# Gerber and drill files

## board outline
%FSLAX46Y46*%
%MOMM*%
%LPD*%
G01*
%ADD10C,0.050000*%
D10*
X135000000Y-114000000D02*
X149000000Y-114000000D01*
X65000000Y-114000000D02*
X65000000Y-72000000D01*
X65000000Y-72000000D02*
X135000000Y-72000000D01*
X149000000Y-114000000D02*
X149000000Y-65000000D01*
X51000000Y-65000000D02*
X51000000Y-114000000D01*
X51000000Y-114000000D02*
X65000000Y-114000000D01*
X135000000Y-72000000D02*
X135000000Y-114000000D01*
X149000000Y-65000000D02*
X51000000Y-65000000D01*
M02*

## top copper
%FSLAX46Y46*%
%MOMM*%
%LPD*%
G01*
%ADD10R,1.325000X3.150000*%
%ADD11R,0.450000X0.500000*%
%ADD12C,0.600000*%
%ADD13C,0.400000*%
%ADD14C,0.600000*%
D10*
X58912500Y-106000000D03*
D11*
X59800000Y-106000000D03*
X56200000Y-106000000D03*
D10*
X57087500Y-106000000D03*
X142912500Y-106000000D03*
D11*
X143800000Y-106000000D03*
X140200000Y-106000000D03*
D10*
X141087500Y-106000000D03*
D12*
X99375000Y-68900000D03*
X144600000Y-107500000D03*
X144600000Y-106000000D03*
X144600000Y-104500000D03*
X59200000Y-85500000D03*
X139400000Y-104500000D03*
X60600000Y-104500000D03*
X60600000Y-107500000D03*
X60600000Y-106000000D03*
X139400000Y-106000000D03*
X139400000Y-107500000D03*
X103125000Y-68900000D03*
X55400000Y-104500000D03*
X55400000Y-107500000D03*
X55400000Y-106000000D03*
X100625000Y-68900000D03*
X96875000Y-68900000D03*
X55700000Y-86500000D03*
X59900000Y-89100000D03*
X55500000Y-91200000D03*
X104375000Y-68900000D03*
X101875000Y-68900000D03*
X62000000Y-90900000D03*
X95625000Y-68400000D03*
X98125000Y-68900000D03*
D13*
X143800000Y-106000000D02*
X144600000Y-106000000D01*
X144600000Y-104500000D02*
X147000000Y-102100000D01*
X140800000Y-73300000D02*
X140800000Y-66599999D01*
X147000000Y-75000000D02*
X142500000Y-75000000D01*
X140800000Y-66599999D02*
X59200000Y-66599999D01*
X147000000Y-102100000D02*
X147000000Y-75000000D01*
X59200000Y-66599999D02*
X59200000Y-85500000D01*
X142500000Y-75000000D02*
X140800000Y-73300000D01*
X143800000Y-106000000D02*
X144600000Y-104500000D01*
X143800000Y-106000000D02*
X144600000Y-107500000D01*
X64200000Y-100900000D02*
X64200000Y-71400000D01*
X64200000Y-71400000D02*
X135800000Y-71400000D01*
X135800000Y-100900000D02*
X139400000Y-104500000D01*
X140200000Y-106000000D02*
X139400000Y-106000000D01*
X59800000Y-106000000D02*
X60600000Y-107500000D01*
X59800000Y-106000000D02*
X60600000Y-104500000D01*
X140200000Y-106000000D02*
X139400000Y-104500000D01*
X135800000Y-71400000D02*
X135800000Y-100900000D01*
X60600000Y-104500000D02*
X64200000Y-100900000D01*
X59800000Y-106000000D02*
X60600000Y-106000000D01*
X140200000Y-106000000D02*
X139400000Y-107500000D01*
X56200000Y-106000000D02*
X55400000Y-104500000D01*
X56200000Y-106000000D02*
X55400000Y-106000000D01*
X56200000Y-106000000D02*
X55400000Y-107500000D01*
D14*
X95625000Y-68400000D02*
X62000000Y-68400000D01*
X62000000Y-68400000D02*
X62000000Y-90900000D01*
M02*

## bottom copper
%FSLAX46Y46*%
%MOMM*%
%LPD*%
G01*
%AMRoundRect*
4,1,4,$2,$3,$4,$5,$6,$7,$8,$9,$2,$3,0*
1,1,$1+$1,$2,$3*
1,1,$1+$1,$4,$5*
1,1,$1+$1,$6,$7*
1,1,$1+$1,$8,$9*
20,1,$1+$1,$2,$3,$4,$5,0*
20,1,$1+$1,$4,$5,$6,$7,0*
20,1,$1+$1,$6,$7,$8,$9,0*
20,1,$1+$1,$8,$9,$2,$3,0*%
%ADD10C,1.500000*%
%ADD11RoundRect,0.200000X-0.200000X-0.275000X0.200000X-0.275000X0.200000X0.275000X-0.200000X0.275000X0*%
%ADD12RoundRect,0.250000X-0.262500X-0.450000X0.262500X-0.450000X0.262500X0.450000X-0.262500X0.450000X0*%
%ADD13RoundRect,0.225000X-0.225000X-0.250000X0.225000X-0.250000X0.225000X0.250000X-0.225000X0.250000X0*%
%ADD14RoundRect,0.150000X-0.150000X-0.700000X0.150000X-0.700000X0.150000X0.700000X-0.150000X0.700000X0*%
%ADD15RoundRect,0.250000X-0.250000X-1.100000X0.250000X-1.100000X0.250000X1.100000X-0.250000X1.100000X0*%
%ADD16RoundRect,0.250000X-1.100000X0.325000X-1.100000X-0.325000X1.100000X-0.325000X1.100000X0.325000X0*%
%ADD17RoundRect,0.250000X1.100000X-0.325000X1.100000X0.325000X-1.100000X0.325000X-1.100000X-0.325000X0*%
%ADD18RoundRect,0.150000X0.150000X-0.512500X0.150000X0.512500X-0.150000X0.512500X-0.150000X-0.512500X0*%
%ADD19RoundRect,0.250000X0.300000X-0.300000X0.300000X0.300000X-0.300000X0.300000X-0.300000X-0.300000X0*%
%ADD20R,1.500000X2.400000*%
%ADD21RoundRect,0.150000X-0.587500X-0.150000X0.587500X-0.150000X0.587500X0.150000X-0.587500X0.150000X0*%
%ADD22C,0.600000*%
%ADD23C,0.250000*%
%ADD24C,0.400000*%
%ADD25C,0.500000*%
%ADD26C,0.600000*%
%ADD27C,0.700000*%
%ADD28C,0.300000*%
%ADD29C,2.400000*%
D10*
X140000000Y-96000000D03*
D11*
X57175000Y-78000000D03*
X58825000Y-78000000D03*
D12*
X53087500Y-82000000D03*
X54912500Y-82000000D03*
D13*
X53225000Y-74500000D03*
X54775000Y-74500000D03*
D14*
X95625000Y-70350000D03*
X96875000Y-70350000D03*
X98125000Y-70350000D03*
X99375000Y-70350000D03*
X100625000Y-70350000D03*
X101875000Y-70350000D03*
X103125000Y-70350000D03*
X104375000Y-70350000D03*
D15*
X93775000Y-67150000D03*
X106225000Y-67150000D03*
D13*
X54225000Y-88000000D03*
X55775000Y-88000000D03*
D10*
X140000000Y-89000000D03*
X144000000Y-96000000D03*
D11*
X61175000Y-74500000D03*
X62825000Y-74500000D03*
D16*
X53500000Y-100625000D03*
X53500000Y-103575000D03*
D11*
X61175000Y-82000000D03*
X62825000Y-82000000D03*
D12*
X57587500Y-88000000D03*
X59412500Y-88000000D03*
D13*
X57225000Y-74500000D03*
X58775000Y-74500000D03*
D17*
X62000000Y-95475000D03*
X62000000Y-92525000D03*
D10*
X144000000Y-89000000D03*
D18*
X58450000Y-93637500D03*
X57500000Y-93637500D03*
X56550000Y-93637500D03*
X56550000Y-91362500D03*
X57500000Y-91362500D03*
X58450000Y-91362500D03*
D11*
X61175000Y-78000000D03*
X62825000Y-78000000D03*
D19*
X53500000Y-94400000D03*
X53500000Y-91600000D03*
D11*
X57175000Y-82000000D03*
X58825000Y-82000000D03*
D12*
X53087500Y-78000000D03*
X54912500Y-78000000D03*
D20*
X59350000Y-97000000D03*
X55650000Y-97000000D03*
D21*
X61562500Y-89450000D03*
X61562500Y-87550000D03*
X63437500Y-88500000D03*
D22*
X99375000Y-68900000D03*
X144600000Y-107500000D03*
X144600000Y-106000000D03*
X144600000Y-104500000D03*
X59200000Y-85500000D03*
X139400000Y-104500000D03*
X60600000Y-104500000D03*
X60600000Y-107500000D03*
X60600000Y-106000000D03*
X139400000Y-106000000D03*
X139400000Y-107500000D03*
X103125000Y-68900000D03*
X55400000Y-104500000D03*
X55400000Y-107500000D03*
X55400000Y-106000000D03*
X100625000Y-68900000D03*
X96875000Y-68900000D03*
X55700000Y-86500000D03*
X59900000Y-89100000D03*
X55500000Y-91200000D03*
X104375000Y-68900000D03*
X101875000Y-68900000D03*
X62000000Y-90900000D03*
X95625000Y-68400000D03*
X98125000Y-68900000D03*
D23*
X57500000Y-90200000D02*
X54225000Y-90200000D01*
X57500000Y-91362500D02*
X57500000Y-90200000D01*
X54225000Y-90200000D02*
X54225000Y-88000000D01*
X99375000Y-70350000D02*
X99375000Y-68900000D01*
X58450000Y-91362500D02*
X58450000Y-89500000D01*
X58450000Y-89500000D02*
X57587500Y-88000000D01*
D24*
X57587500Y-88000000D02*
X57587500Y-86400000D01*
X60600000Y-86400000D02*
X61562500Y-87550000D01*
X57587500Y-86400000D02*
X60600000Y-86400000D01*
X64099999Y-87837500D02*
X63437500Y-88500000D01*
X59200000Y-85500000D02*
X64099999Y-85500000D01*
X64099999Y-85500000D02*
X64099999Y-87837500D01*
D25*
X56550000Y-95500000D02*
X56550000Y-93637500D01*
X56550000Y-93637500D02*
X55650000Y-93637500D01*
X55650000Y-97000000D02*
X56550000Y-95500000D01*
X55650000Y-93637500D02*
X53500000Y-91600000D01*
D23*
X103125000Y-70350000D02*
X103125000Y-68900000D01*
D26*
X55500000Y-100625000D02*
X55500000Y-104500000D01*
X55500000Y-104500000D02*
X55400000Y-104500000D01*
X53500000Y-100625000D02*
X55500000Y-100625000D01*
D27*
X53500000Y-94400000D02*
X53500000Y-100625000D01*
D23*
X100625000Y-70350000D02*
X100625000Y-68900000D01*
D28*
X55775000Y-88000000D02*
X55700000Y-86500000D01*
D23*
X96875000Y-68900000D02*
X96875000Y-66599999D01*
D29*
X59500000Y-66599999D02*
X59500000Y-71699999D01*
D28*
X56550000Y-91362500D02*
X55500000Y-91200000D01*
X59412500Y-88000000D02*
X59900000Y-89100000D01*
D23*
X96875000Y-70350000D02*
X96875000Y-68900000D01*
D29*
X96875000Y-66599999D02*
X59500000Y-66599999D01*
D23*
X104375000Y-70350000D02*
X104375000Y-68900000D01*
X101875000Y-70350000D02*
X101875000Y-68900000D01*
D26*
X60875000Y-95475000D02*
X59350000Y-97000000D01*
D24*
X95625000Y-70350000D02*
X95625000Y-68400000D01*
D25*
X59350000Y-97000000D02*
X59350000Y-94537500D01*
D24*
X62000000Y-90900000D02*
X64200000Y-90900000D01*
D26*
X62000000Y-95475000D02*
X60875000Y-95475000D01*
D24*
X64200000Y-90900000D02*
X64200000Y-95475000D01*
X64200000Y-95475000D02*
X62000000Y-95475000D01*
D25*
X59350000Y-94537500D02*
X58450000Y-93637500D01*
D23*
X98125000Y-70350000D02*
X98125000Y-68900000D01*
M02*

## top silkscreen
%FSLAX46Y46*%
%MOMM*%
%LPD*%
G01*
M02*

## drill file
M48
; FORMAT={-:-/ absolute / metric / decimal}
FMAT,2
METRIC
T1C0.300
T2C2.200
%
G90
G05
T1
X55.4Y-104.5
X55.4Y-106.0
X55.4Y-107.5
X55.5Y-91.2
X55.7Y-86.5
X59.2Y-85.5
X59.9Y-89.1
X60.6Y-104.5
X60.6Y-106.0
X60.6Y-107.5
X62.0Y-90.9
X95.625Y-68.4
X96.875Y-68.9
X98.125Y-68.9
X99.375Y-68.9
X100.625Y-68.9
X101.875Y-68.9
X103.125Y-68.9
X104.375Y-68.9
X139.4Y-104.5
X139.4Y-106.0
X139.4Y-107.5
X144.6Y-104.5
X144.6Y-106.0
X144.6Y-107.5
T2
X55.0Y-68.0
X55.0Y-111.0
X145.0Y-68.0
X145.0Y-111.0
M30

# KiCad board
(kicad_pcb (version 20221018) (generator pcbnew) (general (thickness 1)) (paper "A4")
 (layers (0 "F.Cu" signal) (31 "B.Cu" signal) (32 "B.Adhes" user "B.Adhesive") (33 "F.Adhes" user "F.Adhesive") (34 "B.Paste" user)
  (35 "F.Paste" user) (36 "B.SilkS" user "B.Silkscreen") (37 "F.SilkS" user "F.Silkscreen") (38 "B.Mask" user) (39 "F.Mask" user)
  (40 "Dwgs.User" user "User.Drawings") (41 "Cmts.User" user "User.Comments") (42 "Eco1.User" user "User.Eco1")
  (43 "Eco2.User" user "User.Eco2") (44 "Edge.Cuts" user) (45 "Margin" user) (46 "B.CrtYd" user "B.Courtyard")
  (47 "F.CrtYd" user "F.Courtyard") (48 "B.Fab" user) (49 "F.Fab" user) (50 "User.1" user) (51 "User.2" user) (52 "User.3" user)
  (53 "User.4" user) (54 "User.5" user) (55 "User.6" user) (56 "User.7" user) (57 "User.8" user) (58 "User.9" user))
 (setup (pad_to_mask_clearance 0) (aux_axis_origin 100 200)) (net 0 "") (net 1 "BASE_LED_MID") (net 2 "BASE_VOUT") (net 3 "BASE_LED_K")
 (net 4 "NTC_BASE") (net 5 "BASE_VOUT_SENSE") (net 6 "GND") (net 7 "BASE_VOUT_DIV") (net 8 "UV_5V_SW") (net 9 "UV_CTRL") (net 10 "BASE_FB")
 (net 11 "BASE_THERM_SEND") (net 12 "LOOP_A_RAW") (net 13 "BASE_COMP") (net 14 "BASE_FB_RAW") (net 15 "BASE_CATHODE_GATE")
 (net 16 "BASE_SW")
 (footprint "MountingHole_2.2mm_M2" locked (layer "F.Cu") (at 55 68)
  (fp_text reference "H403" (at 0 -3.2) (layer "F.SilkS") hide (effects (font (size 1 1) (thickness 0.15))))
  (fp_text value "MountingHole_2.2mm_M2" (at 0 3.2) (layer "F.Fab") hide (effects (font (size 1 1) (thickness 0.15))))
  (pad "" np_thru_hole circle locked (at 0 0) (size 2.2 2.2) (drill 2.2) (layers "*.Cu" "*.Mask")))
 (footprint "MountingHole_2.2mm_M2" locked (layer "F.Cu") (at 145 111)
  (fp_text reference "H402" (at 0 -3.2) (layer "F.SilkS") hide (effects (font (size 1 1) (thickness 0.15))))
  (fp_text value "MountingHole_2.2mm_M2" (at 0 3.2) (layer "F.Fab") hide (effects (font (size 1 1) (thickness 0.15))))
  (pad "" np_thru_hole circle locked (at 0 0) (size 2.2 2.2) (drill 2.2) (layers "*.Cu" "*.Mask")))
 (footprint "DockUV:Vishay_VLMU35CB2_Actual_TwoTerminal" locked (layer "F.Cu") (at 58 106)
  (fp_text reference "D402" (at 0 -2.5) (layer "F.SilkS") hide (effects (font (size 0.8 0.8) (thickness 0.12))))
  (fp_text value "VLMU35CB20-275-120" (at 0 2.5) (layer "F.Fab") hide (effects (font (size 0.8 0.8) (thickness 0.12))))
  (pad "1" smd rect locked (at 0.9125 0) (size 1.325 3.15) (layers "F.Cu" "F.Paste" "F.Mask") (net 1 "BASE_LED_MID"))
  (pad "1" smd rect locked (at 1.8 0) (size 0.45 0.5) (layers "F.Cu" "F.Paste" "F.Mask") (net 1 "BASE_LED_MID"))
  (pad "2" smd rect locked (at -1.8 0) (size 0.45 0.5) (layers "F.Cu" "F.Paste" "F.Mask") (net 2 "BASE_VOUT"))
  (pad "2" smd rect locked (at -0.9125 0) (size 1.325 3.15) (layers "F.Cu" "F.Paste" "F.Mask") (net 2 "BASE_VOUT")))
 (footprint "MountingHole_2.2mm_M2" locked (layer "F.Cu") (at 55 111)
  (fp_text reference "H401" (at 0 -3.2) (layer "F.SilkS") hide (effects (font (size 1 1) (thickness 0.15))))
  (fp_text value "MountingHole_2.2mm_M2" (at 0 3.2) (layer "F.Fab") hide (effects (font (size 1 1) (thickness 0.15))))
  (pad "" np_thru_hole circle locked (at 0 0) (size 2.2 2.2) (drill 2.2) (layers "*.Cu" "*.Mask")))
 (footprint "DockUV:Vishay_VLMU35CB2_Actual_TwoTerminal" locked (layer "F.Cu") (at 142 106)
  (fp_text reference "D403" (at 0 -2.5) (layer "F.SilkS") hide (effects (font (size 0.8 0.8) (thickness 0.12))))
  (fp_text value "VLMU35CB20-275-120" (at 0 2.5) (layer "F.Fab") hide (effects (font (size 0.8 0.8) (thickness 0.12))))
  (pad "1" smd rect locked (at 0.9125 0) (size 1.325 3.15) (layers "F.Cu" "F.Paste" "F.Mask") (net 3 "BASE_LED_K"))
  (pad "1" smd rect locked (at 1.8 0) (size 0.45 0.5) (layers "F.Cu" "F.Paste" "F.Mask") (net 3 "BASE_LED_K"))
  (pad "2" smd rect locked (at -1.8 0) (size 0.45 0.5) (layers "F.Cu" "F.Paste" "F.Mask") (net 1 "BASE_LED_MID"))
  (pad "2" smd rect locked (at -0.9125 0) (size 1.325 3.15) (layers "F.Cu" "F.Paste" "F.Mask") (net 1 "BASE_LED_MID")))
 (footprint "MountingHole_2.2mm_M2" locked (layer "F.Cu") (at 145 68)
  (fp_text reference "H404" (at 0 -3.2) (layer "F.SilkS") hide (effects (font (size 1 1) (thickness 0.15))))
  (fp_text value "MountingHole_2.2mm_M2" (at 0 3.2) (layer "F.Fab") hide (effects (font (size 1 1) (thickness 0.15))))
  (pad "" np_thru_hole circle locked (at 0 0) (size 2.2 2.2) (drill 2.2) (layers "*.Cu" "*.Mask")))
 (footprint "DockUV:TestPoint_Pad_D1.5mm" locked (layer "B.Cu") (at 140 96)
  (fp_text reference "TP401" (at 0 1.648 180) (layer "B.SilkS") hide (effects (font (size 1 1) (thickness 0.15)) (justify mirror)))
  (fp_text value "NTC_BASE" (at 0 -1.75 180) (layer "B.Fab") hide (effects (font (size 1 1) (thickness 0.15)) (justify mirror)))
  (pad "1" smd circle locked (at 0 0) (size 1.5 1.5) (layers "B.Cu" "B.Mask") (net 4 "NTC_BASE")))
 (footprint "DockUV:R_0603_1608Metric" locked (layer "B.Cu") (at 58 78)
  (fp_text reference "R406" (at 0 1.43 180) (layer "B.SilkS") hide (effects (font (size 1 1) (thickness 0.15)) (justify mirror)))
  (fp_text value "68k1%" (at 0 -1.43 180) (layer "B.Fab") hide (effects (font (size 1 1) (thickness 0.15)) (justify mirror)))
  (pad "1" smd roundrect locked (at -0.825 0) (size 0.8 0.95) (layers "B.Cu" "B.Paste" "B.Mask") (roundrect_rratio 0.25)
   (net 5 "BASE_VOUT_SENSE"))
  (pad "2" smd roundrect locked (at 0.825 0) (size 0.8 0.95) (layers "B.Cu" "B.Paste" "B.Mask") (roundrect_rratio 0.25) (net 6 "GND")))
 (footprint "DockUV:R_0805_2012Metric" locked (layer "B.Cu") (at 54 82)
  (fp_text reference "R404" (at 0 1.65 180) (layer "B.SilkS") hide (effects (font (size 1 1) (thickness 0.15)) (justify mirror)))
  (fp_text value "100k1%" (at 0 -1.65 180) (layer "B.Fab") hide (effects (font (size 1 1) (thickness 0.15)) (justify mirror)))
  (pad "1" smd roundrect locked (at -0.9125 0) (size 1.025 1.4) (layers "B.Cu" "B.Paste" "B.Mask") (roundrect_rratio 0.243902)
   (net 2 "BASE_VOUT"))
  (pad "2" smd roundrect locked (at 0.9125 0) (size 1.025 1.4) (layers "B.Cu" "B.Paste" "B.Mask") (roundrect_rratio 0.243902) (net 6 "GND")))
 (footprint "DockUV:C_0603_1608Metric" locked (layer "B.Cu") (at 54 74.5)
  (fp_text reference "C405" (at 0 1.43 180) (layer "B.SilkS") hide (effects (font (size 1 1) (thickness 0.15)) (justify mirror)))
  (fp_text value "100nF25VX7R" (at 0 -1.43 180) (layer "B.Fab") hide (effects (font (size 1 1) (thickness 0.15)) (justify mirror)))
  (pad "1" smd roundrect locked (at -0.775 0) (size 0.9 0.95) (layers "B.Cu" "B.Paste" "B.Mask") (roundrect_rratio 0.25)
   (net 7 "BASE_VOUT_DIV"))
  (pad "2" smd roundrect locked (at 0.775 0) (size 0.9 0.95) (layers "B.Cu" "B.Paste" "B.Mask") (roundrect_rratio 0.25) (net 6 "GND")))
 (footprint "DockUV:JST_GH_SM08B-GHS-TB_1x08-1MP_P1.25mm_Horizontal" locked (layer "B.Cu") (at 100 68.5)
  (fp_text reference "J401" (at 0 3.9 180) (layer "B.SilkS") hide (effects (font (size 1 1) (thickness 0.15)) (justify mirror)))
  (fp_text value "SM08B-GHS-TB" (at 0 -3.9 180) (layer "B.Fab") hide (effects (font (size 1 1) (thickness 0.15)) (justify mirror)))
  (pad "1" smd roundrect locked (at -4.375 1.85) (size 0.6 1.7) (layers "B.Cu" "B.Paste" "B.Mask") (roundrect_rratio 0.25)
   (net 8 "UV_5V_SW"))
  (pad "2" smd roundrect locked (at -3.125 1.85) (size 0.6 1.7) (layers "B.Cu" "B.Paste" "B.Mask") (roundrect_rratio 0.25) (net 6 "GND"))
  (pad "3" smd roundrect locked (at -1.875 1.85) (size 0.6 1.7) (layers "B.Cu" "B.Paste" "B.Mask") (roundrect_rratio 0.25) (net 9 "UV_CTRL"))
  (pad "4" smd roundrect locked (at -0.625 1.85) (size 0.6 1.7) (layers "B.Cu" "B.Paste" "B.Mask") (roundrect_rratio 0.25)
   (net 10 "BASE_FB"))
  (pad "5" smd roundrect locked (at 0.625 1.85) (size 0.6 1.7) (layers "B.Cu" "B.Paste" "B.Mask") (roundrect_rratio 0.25)
   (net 7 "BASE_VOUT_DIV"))
  (pad "6" smd roundrect locked (at 1.875 1.85) (size 0.6 1.7) (layers "B.Cu" "B.Paste" "B.Mask") (roundrect_rratio 0.25) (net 4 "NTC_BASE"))
  (pad "7" smd roundrect locked (at 3.125 1.85) (size 0.6 1.7) (layers "B.Cu" "B.Paste" "B.Mask") (roundrect_rratio 0.25)
   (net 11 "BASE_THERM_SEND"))
  (pad "8" smd roundrect locked (at 4.375 1.85) (size 0.6 1.7) (layers "B.Cu" "B.Paste" "B.Mask") (roundrect_rratio 0.25)
   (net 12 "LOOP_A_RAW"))
  (pad "MP" smd roundrect locked (at -6.225 -1.35) (size 1 2.7) (layers "B.Cu" "B.Paste" "B.Mask") (roundrect_rratio 0.25) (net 6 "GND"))
  (pad "MP" smd roundrect locked (at 6.225 -1.35) (size 1 2.7) (layers "B.Cu" "B.Paste" "B.Mask") (roundrect_rratio 0.25) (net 6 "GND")))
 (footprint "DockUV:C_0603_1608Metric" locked (layer "B.Cu") (at 55 88)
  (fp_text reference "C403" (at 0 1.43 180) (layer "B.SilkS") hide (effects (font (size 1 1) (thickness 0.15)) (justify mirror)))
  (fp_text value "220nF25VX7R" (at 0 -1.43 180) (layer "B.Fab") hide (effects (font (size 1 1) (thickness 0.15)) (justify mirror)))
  (pad "1" smd roundrect locked (at -0.775 0) (size 0.9 0.95) (layers "B.Cu" "B.Paste" "B.Mask") (roundrect_rratio 0.25)
   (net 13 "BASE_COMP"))
  (pad "2" smd roundrect locked (at 0.775 0) (size 0.9 0.95) (layers "B.Cu" "B.Paste" "B.Mask") (roundrect_rratio 0.25) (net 6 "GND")))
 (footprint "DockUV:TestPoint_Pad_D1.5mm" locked (layer "B.Cu") (at 140 89)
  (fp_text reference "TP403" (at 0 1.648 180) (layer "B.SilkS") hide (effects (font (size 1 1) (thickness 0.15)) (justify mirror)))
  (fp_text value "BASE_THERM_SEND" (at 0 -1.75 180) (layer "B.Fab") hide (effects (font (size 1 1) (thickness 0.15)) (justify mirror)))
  (pad "1" smd circle locked (at 0 0) (size 1.5 1.5) (layers "B.Cu" "B.Mask") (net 11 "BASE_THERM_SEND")))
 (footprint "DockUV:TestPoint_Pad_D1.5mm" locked (layer "B.Cu") (at 144 96)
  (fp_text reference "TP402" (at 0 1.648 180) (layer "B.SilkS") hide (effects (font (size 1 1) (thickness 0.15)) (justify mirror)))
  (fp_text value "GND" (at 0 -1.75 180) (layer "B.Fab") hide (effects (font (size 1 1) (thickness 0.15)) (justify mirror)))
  (pad "1" smd circle locked (at 0 0) (size 1.5 1.5) (layers "B.Cu" "B.Mask") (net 6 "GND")))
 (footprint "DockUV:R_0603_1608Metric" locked (layer "B.Cu") (at 62 74.5)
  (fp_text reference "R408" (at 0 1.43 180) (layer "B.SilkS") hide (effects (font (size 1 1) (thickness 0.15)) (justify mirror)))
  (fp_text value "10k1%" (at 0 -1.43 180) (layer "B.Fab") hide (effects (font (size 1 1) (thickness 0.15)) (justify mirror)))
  (pad "1" smd roundrect locked (at -0.825 0) (size 0.8 0.95) (layers "B.Cu" "B.Paste" "B.Mask") (roundrect_rratio 0.25)
   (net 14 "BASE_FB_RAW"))
  (pad "2" smd roundrect locked (at 0.825 0) (size 0.8 0.95) (layers "B.Cu" "B.Paste" "B.Mask") (roundrect_rratio 0.25) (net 10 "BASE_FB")))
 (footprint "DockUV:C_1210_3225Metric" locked (layer "B.Cu") (at 53.5 102.1 -90)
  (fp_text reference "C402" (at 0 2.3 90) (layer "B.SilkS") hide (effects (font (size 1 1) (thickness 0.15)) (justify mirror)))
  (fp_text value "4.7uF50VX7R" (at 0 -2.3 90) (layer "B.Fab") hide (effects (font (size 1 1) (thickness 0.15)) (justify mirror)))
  (pad "1" smd roundrect locked (at -1.475 0 270) (size 1.15 2.7) (layers "B.Cu" "B.Paste" "B.Mask") (roundrect_rratio 0.217391)
   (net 2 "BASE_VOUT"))
  (pad "2" smd roundrect locked (at 1.475 0 270) (size 1.15 2.7) (layers "B.Cu" "B.Paste" "B.Mask") (roundrect_rratio 0.217391)
   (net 6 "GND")))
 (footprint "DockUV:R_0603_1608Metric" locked (layer "B.Cu") (at 62 82)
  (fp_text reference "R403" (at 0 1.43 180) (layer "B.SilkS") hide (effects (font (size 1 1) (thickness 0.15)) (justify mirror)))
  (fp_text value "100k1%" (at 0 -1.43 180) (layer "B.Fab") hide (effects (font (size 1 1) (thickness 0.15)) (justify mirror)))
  (pad "1" smd roundrect locked (at -0.825 0) (size 0.8 0.95) (layers "B.Cu" "B.Paste" "B.Mask") (roundrect_rratio 0.25)
   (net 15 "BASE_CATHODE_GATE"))
  (pad "2" smd roundrect locked (at 0.825 0) (size 0.8 0.95) (layers "B.Cu" "B.Paste" "B.Mask") (roundrect_rratio 0.25) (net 6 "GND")))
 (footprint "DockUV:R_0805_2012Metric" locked (layer "B.Cu") (at 58.5 88)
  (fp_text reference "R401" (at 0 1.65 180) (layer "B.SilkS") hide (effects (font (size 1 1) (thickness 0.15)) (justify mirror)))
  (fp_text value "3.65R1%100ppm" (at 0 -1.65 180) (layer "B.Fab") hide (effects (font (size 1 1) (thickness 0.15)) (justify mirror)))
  (pad "1" smd roundrect locked (at -0.9125 0) (size 1.025 1.4) (layers "B.Cu" "B.Paste" "B.Mask") (roundrect_rratio 0.243902)
   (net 14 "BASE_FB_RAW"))
  (pad "2" smd roundrect locked (at 0.9125 0) (size 1.025 1.4) (layers "B.Cu" "B.Paste" "B.Mask") (roundrect_rratio 0.243902) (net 6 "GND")))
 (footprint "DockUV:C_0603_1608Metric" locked (layer "B.Cu") (at 58 74.5)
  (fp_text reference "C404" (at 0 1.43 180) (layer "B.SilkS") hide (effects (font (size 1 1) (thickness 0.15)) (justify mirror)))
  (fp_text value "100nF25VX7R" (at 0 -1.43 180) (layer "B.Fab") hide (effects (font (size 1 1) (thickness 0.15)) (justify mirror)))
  (pad "1" smd roundrect locked (at -0.775 0) (size 0.9 0.95) (layers "B.Cu" "B.Paste" "B.Mask") (roundrect_rratio 0.25) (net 10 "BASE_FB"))
  (pad "2" smd roundrect locked (at 0.775 0) (size 0.9 0.95) (layers "B.Cu" "B.Paste" "B.Mask") (roundrect_rratio 0.25) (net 6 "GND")))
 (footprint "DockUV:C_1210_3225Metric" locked (layer "B.Cu") (at 62 94 90)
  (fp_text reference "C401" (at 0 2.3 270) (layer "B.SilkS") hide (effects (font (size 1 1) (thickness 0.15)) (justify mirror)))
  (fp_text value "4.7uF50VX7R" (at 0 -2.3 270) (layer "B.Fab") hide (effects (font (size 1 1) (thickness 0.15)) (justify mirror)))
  (pad "1" smd roundrect locked (at -1.475 0 90) (size 1.15 2.7) (layers "B.Cu" "B.Paste" "B.Mask") (roundrect_rratio 0.217391)
   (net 8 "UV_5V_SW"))
  (pad "2" smd roundrect locked (at 1.475 0 90) (size 1.15 2.7) (layers "B.Cu" "B.Paste" "B.Mask") (roundrect_rratio 0.217391) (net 6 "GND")))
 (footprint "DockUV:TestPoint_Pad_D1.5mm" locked (layer "B.Cu") (at 144 89)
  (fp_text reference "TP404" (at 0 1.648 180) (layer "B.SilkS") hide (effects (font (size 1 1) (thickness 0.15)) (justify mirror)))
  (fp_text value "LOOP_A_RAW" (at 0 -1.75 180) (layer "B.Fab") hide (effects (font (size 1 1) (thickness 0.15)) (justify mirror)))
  (pad "1" smd circle locked (at 0 0) (size 1.5 1.5) (layers "B.Cu" "B.Mask") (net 12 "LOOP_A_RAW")))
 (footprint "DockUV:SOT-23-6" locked (layer "B.Cu") (at 57.5 92.5 90)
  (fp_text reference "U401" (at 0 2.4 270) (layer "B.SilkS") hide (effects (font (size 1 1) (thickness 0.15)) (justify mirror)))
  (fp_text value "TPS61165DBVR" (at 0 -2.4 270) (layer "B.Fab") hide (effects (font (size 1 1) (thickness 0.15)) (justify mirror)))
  (pad "1" smd roundrect locked (at -1.1375 0.95 90) (size 1.325 0.6) (layers "B.Cu" "B.Paste" "B.Mask") (roundrect_rratio 0.25)
   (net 8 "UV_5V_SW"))
  (pad "2" smd roundrect locked (at -1.1375 0 90) (size 1.325 0.6) (layers "B.Cu" "B.Paste" "B.Mask") (roundrect_rratio 0.25)
   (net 9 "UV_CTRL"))
  (pad "3" smd roundrect locked (at -1.1375 -0.95 90) (size 1.325 0.6) (layers "B.Cu" "B.Paste" "B.Mask") (roundrect_rratio 0.25)
   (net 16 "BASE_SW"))
  (pad "4" smd roundrect locked (at 1.1375 -0.95 90) (size 1.325 0.6) (layers "B.Cu" "B.Paste" "B.Mask") (roundrect_rratio 0.25)
   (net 6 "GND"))
  (pad "5" smd roundrect locked (at 1.1375 0 90) (size 1.325 0.6) (layers "B.Cu" "B.Paste" "B.Mask") (roundrect_rratio 0.25)
   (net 13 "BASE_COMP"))
  (pad "6" smd roundrect locked (at 1.1375 0.95 90) (size 1.325 0.6) (layers "B.Cu" "B.Paste" "B.Mask") (roundrect_rratio 0.25)
   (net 14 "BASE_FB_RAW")))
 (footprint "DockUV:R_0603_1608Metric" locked (layer "B.Cu") (at 62 78)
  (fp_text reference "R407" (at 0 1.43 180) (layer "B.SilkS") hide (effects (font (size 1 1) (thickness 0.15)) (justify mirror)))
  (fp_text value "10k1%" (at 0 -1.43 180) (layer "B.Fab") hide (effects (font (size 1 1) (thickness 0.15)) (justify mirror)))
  (pad "1" smd roundrect locked (at -0.825 0) (size 0.8 0.95) (layers "B.Cu" "B.Paste" "B.Mask") (roundrect_rratio 0.25)
   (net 5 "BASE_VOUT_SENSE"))
  (pad "2" smd roundrect locked (at 0.825 0) (size 0.8 0.95) (layers "B.Cu" "B.Paste" "B.Mask") (roundrect_rratio 0.25)
   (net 7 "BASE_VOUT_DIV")))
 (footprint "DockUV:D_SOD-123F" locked (layer "B.Cu") (at 53.5 93 90)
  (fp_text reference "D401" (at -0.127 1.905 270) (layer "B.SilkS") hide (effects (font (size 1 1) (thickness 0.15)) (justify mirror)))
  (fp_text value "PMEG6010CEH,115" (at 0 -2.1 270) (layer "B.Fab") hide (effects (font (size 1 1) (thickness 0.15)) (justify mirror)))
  (pad "1" smd roundrect locked (at -1.4 0 90) (size 1.1 1.1) (layers "B.Cu" "B.Paste" "B.Mask") (roundrect_rratio 0.2272727273)
   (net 2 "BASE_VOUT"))
  (pad "2" smd roundrect locked (at 1.4 0 90) (size 1.1 1.1) (layers "B.Cu" "B.Paste" "B.Mask") (roundrect_rratio 0.2272727273)
   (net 16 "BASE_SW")))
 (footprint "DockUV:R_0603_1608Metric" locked (layer "B.Cu") (at 58 82)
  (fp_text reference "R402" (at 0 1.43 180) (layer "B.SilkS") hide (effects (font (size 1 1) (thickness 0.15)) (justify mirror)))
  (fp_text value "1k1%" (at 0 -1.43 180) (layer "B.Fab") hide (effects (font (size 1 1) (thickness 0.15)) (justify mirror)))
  (pad "1" smd roundrect locked (at -0.825 0) (size 0.8 0.95) (layers "B.Cu" "B.Paste" "B.Mask") (roundrect_rratio 0.25) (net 9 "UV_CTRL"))
  (pad "2" smd roundrect locked (at 0.825 0) (size 0.8 0.95) (layers "B.Cu" "B.Paste" "B.Mask") (roundrect_rratio 0.25)
   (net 15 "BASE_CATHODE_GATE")))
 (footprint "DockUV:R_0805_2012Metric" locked (layer "B.Cu") (at 54 78)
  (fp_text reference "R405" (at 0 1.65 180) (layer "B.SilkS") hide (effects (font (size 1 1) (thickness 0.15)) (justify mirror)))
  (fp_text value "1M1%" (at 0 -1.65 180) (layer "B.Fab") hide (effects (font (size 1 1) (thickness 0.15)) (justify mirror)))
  (pad "1" smd roundrect locked (at -0.9125 0) (size 1.025 1.4) (layers "B.Cu" "B.Paste" "B.Mask") (roundrect_rratio 0.243902)
   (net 2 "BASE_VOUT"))
  (pad "2" smd roundrect locked (at 0.9125 0) (size 1.025 1.4) (layers "B.Cu" "B.Paste" "B.Mask") (roundrect_rratio 0.243902)
   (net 5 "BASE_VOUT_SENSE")))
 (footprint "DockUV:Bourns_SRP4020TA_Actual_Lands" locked (layer "B.Cu") (at 57.5 97 180)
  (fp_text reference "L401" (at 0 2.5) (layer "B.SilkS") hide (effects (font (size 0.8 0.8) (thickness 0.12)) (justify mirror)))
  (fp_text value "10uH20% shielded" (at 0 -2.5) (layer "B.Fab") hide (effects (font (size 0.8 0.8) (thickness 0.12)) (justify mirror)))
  (pad "1" smd rect locked (at -1.85 0 180) (size 1.5 2.4) (layers "B.Cu" "B.Paste" "B.Mask") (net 8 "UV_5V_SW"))
  (pad "2" smd rect locked (at 1.85 0 180) (size 1.5 2.4) (layers "B.Cu" "B.Paste" "B.Mask") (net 16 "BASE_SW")))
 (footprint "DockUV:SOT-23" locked (layer "B.Cu") (at 62.5 88.5)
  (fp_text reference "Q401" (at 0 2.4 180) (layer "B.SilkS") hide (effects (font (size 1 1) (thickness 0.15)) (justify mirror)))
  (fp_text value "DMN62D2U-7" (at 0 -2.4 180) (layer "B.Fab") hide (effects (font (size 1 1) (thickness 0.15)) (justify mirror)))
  (pad "1" smd roundrect locked (at -0.9375 0.95) (size 1.475 0.6) (layers "B.Cu" "B.Paste" "B.Mask") (roundrect_rratio 0.25)
   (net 15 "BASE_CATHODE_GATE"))
  (pad "2" smd roundrect locked (at -0.9375 -0.95) (size 1.475 0.6) (layers "B.Cu" "B.Paste" "B.Mask") (roundrect_rratio 0.25)
   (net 14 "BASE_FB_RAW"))
  (pad "3" smd roundrect locked (at 0.9375 0) (size 1.475 0.6) (layers "B.Cu" "B.Paste" "B.Mask") (roundrect_rratio 0.25)
   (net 3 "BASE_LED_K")))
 (gr_line (start 135 114) (end 149 114) (stroke (width 0.05) (type default)) (layer "Edge.Cuts"))
 (gr_line (start 65 114) (end 65 72) (stroke (width 0.05) (type default)) (layer "Edge.Cuts"))
 (gr_line (start 65 72) (end 135 72) (stroke (width 0.05) (type default)) (layer "Edge.Cuts"))
 (gr_line (start 149 114) (end 149 65) (stroke (width 0.05) (type default)) (layer "Edge.Cuts"))
 (gr_line (start 51 65) (end 51 114) (stroke (width 0.05) (type default)) (layer "Edge.Cuts"))
 (gr_line (start 51 114) (end 65 114) (stroke (width 0.05) (type default)) (layer "Edge.Cuts"))
 (gr_line (start 135 72) (end 135 114) (stroke (width 0.05) (type default)) (layer "Edge.Cuts"))
 (gr_line (start 149 65) (end 51 65) (stroke (width 0.05) (type default)) (layer "Edge.Cuts"))
 (segment locked (start 57.5 90.2) (end 54.225 90.2) (width 0.25) (layer "B.Cu") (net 13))
 (segment locked (start 57.5 91.3625) (end 57.5 90.2) (width 0.25) (layer "B.Cu") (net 13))
 (segment locked (start 54.225 90.2) (end 54.225 88) (width 0.25) (layer "B.Cu") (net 13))
 (via locked (at 99.375 68.9) (size 0.6) (drill 0.3) (layers "F.Cu" "B.Cu") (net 10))
 (segment locked (start 99.375 70.35) (end 99.375 68.9) (width 0.25) (layer "B.Cu") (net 10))
 (segment locked (start 58.45 91.3625) (end 58.45 89.5) (width 0.25) (layer "B.Cu") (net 14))
 (segment locked (start 58.45 89.5) (end 57.5875 88) (width 0.25) (layer "B.Cu") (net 14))
 (segment locked (start 57.5875 88) (end 57.5875 86.4) (width 0.4) (layer "B.Cu") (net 14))
 (segment locked (start 60.6 86.4) (end 61.5625 87.55) (width 0.4) (layer "B.Cu") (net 14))
 (segment locked (start 57.5875 86.4) (end 60.6 86.4) (width 0.4) (layer "B.Cu") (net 14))
 (segment locked (start 143.8 106) (end 144.6 106) (width 0.4) (layer "F.Cu") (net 3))
 (segment locked (start 144.6 104.5) (end 147 102.1) (width 0.4) (layer "F.Cu") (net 3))
 (segment locked (start 140.8 73.3) (end 140.8 66.599999) (width 0.4) (layer "F.Cu") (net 3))
 (segment locked (start 147 75) (end 142.5 75) (width 0.4) (layer "F.Cu") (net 3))
 (segment locked (start 140.8 66.599999) (end 59.2 66.599999) (width 0.4) (layer "F.Cu") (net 3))
 (segment locked (start 147 102.1) (end 147 75) (width 0.4) (layer "F.Cu") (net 3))
 (segment locked (start 59.2 66.599999) (end 59.2 85.5) (width 0.4) (layer "F.Cu") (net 3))
 (segment locked (start 142.5 75) (end 140.8 73.3) (width 0.4) (layer "F.Cu") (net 3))
 (segment locked (start 143.8 106) (end 144.6 104.5) (width 0.4) (layer "F.Cu") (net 3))
 (segment locked (start 143.8 106) (end 144.6 107.5) (width 0.4) (layer "F.Cu") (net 3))
 (via locked (at 144.6 107.5) (size 0.6) (drill 0.3) (layers "F.Cu" "B.Cu") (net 3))
 (via locked (at 144.6 106) (size 0.6) (drill 0.3) (layers "F.Cu" "B.Cu") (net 3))
 (via locked (at 144.6 104.5) (size 0.6) (drill 0.3) (layers "F.Cu" "B.Cu") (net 3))
 (via locked (at 59.2 85.5) (size 0.6) (drill 0.3) (layers "F.Cu" "B.Cu") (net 3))
 (segment locked (start 64.099999 87.8375) (end 63.4375 88.5) (width 0.4) (layer "B.Cu") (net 3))
 (segment locked (start 59.2 85.5) (end 64.099999 85.5) (width 0.4) (layer "B.Cu") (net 3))
 (segment locked (start 64.099999 85.5) (end 64.099999 87.8375) (width 0.4) (layer "B.Cu") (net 3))
 (segment locked (start 64.2 100.9) (end 64.2 71.4) (width 0.4) (layer "F.Cu") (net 1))
 (segment locked (start 64.2 71.4) (end 135.8 71.4) (width 0.4) (layer "F.Cu") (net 1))
 (segment locked (start 135.8 100.9) (end 139.4 104.5) (width 0.4) (layer "F.Cu") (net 1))
 (segment locked (start 140.2 106) (end 139.4 106) (width 0.4) (layer "F.Cu") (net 1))
 (segment locked (start 59.8 106) (end 60.6 107.5) (width 0.4) (layer "F.Cu") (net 1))
 (segment locked (start 59.8 106) (end 60.6 104.5) (width 0.4) (layer "F.Cu") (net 1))
 (segment locked (start 140.2 106) (end 139.4 104.5) (width 0.4) (layer "F.Cu") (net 1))
 (segment locked (start 135.8 71.4) (end 135.8 100.9) (width 0.4) (layer "F.Cu") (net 1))
 (segment locked (start 60.6 104.5) (end 64.2 100.9) (width 0.4) (layer "F.Cu") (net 1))
 (segment locked (start 59.8 106) (end 60.6 106) (width 0.4) (layer "F.Cu") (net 1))
 (segment locked (start 140.2 106) (end 139.4 107.5) (width 0.4) (layer "F.Cu") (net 1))
 (via locked (at 139.4 104.5) (size 0.6) (drill 0.3) (layers "F.Cu" "B.Cu") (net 1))
 (via locked (at 60.6 104.5) (size 0.6) (drill 0.3) (layers "F.Cu" "B.Cu") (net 1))
 (via locked (at 60.6 107.5) (size 0.6) (drill 0.3) (layers "F.Cu" "B.Cu") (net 1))
 (via locked (at 60.6 106) (size 0.6) (drill 0.3) (layers "F.Cu" "B.Cu") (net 1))
 (via locked (at 139.4 106) (size 0.6) (drill 0.3) (layers "F.Cu" "B.Cu") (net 1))
 (via locked (at 139.4 107.5) (size 0.6) (drill 0.3) (layers "F.Cu" "B.Cu") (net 1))
 (segment locked (start 56.55 95.5) (end 56.55 93.6375) (width 0.5) (layer "B.Cu") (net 16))
 (segment locked (start 56.55 93.6375) (end 55.65 93.6375) (width 0.5) (layer "B.Cu") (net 16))
 (segment locked (start 55.65 97) (end 56.55 95.5) (width 0.5) (layer "B.Cu") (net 16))
 (segment locked (start 55.65 93.6375) (end 53.5 91.6) (width 0.5) (layer "B.Cu") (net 16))
 (via locked (at 103.125 68.9) (size 0.6) (drill 0.3) (layers "F.Cu" "B.Cu") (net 11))
 (segment locked (start 103.125 70.35) (end 103.125 68.9) (width 0.25) (layer "B.Cu") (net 11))
 (segment locked (start 56.2 106) (end 55.4 104.5) (width 0.4) (layer "F.Cu") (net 2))
 (segment locked (start 56.2 106) (end 55.4 106) (width 0.4) (layer "F.Cu") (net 2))
 (segment locked (start 56.2 106) (end 55.4 107.5) (width 0.4) (layer "F.Cu") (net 2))
 (via locked (at 55.4 104.5) (size 0.6) (drill 0.3) (layers "F.Cu" "B.Cu") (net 2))
 (via locked (at 55.4 107.5) (size 0.6) (drill 0.3) (layers "F.Cu" "B.Cu") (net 2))
 (via locked (at 55.4 106) (size 0.6) (drill 0.3) (layers "F.Cu" "B.Cu") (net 2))
 (segment locked (start 55.5 100.625) (end 55.5 104.5) (width 0.6) (layer "B.Cu") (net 2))
 (segment locked (start 55.5 104.5) (end 55.4 104.5) (width 0.6) (layer "B.Cu") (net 2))
 (segment locked (start 53.5 100.625) (end 55.5 100.625) (width 0.6) (layer "B.Cu") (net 2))
 (segment locked (start 53.5 94.4) (end 53.5 100.625) (width 0.7) (layer "B.Cu") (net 2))
 (via locked (at 100.625 68.9) (size 0.6) (drill 0.3) (layers "F.Cu" "B.Cu") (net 7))
 (segment locked (start 100.625 70.35) (end 100.625 68.9) (width 0.25) (layer "B.Cu") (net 7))
 (via locked (at 96.875 68.9) (size 0.6) (drill 0.3) (layers "F.Cu" "B.Cu") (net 6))
 (via locked (at 55.7 86.5) (size 0.6) (drill 0.3) (layers "F.Cu" "B.Cu") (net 6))
 (via locked (at 59.9 89.1) (size 0.6) (drill 0.3) (layers "F.Cu" "B.Cu") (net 6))
 (via locked (at 55.5 91.2) (size 0.6) (drill 0.3) (layers "F.Cu" "B.Cu") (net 6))
 (segment locked (start 55.775 88) (end 55.7 86.5) (width 0.3) (layer "B.Cu") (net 6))
 (segment locked (start 96.875 68.9) (end 96.875 66.599999) (width 0.25) (layer "B.Cu") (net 6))
 (segment locked (start 59.5 66.599999) (end 59.5 71.699999) (width 2.4) (layer "B.Cu") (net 6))
 (segment locked (start 56.55 91.3625) (end 55.5 91.2) (width 0.3) (layer "B.Cu") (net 6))
 (segment locked (start 59.4125 88) (end 59.9 89.1) (width 0.3) (layer "B.Cu") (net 6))
 (segment locked (start 96.875 70.35) (end 96.875 68.9) (width 0.25) (layer "B.Cu") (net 6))
 (segment locked (start 96.875 66.599999) (end 59.5 66.599999) (width 2.4) (layer "B.Cu") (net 6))
 (via locked (at 104.375 68.9) (size 0.6) (drill 0.3) (layers "F.Cu" "B.Cu") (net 12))
 (segment locked (start 104.375 70.35) (end 104.375 68.9) (width 0.25) (layer "B.Cu") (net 12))
 (via locked (at 101.875 68.9) (size 0.6) (drill 0.3) (layers "F.Cu" "B.Cu") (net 4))
 (segment locked (start 101.875 70.35) (end 101.875 68.9) (width 0.25) (layer "B.Cu") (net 4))
 (segment locked (start 95.625 68.4) (end 62 68.4) (width 0.6) (layer "F.Cu") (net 8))
 (segment locked (start 62 68.4) (end 62 90.9) (width 0.6) (layer "F.Cu") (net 8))
 (via locked (at 62 90.9) (size 0.6) (drill 0.3) (layers "F.Cu" "B.Cu") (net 8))
 (via locked (at 95.625 68.4) (size 0.6) (drill 0.3) (layers "F.Cu" "B.Cu") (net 8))
 (segment locked (start 60.875 95.475) (end 59.35 97) (width 0.6) (layer "B.Cu") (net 8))
 (segment locked (start 95.625 70.35) (end 95.625 68.4) (width 0.4) (layer "B.Cu") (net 8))
 (segment locked (start 59.35 97) (end 59.35 94.5375) (width 0.5) (layer "B.Cu") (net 8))
 (segment locked (start 62 90.9) (end 64.2 90.9) (width 0.4) (layer "B.Cu") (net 8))
 (segment locked (start 62 95.475) (end 60.875 95.475) (width 0.6) (layer "B.Cu") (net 8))
 (segment locked (start 64.2 90.9) (end 64.2 95.475) (width 0.4) (layer "B.Cu") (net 8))
 (segment locked (start 64.2 95.475) (end 62 95.475) (width 0.4) (layer "B.Cu") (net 8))
 (segment locked (start 59.35 94.5375) (end 58.45 93.6375) (width 0.5) (layer "B.Cu") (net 8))
 (via locked (at 98.125 68.9) (size 0.6) (drill 0.3) (layers "F.Cu" "B.Cu") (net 9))
 (segment locked (start 98.125 70.35) (end 98.125 68.9) (width 0.25) (layer "B.Cu") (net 9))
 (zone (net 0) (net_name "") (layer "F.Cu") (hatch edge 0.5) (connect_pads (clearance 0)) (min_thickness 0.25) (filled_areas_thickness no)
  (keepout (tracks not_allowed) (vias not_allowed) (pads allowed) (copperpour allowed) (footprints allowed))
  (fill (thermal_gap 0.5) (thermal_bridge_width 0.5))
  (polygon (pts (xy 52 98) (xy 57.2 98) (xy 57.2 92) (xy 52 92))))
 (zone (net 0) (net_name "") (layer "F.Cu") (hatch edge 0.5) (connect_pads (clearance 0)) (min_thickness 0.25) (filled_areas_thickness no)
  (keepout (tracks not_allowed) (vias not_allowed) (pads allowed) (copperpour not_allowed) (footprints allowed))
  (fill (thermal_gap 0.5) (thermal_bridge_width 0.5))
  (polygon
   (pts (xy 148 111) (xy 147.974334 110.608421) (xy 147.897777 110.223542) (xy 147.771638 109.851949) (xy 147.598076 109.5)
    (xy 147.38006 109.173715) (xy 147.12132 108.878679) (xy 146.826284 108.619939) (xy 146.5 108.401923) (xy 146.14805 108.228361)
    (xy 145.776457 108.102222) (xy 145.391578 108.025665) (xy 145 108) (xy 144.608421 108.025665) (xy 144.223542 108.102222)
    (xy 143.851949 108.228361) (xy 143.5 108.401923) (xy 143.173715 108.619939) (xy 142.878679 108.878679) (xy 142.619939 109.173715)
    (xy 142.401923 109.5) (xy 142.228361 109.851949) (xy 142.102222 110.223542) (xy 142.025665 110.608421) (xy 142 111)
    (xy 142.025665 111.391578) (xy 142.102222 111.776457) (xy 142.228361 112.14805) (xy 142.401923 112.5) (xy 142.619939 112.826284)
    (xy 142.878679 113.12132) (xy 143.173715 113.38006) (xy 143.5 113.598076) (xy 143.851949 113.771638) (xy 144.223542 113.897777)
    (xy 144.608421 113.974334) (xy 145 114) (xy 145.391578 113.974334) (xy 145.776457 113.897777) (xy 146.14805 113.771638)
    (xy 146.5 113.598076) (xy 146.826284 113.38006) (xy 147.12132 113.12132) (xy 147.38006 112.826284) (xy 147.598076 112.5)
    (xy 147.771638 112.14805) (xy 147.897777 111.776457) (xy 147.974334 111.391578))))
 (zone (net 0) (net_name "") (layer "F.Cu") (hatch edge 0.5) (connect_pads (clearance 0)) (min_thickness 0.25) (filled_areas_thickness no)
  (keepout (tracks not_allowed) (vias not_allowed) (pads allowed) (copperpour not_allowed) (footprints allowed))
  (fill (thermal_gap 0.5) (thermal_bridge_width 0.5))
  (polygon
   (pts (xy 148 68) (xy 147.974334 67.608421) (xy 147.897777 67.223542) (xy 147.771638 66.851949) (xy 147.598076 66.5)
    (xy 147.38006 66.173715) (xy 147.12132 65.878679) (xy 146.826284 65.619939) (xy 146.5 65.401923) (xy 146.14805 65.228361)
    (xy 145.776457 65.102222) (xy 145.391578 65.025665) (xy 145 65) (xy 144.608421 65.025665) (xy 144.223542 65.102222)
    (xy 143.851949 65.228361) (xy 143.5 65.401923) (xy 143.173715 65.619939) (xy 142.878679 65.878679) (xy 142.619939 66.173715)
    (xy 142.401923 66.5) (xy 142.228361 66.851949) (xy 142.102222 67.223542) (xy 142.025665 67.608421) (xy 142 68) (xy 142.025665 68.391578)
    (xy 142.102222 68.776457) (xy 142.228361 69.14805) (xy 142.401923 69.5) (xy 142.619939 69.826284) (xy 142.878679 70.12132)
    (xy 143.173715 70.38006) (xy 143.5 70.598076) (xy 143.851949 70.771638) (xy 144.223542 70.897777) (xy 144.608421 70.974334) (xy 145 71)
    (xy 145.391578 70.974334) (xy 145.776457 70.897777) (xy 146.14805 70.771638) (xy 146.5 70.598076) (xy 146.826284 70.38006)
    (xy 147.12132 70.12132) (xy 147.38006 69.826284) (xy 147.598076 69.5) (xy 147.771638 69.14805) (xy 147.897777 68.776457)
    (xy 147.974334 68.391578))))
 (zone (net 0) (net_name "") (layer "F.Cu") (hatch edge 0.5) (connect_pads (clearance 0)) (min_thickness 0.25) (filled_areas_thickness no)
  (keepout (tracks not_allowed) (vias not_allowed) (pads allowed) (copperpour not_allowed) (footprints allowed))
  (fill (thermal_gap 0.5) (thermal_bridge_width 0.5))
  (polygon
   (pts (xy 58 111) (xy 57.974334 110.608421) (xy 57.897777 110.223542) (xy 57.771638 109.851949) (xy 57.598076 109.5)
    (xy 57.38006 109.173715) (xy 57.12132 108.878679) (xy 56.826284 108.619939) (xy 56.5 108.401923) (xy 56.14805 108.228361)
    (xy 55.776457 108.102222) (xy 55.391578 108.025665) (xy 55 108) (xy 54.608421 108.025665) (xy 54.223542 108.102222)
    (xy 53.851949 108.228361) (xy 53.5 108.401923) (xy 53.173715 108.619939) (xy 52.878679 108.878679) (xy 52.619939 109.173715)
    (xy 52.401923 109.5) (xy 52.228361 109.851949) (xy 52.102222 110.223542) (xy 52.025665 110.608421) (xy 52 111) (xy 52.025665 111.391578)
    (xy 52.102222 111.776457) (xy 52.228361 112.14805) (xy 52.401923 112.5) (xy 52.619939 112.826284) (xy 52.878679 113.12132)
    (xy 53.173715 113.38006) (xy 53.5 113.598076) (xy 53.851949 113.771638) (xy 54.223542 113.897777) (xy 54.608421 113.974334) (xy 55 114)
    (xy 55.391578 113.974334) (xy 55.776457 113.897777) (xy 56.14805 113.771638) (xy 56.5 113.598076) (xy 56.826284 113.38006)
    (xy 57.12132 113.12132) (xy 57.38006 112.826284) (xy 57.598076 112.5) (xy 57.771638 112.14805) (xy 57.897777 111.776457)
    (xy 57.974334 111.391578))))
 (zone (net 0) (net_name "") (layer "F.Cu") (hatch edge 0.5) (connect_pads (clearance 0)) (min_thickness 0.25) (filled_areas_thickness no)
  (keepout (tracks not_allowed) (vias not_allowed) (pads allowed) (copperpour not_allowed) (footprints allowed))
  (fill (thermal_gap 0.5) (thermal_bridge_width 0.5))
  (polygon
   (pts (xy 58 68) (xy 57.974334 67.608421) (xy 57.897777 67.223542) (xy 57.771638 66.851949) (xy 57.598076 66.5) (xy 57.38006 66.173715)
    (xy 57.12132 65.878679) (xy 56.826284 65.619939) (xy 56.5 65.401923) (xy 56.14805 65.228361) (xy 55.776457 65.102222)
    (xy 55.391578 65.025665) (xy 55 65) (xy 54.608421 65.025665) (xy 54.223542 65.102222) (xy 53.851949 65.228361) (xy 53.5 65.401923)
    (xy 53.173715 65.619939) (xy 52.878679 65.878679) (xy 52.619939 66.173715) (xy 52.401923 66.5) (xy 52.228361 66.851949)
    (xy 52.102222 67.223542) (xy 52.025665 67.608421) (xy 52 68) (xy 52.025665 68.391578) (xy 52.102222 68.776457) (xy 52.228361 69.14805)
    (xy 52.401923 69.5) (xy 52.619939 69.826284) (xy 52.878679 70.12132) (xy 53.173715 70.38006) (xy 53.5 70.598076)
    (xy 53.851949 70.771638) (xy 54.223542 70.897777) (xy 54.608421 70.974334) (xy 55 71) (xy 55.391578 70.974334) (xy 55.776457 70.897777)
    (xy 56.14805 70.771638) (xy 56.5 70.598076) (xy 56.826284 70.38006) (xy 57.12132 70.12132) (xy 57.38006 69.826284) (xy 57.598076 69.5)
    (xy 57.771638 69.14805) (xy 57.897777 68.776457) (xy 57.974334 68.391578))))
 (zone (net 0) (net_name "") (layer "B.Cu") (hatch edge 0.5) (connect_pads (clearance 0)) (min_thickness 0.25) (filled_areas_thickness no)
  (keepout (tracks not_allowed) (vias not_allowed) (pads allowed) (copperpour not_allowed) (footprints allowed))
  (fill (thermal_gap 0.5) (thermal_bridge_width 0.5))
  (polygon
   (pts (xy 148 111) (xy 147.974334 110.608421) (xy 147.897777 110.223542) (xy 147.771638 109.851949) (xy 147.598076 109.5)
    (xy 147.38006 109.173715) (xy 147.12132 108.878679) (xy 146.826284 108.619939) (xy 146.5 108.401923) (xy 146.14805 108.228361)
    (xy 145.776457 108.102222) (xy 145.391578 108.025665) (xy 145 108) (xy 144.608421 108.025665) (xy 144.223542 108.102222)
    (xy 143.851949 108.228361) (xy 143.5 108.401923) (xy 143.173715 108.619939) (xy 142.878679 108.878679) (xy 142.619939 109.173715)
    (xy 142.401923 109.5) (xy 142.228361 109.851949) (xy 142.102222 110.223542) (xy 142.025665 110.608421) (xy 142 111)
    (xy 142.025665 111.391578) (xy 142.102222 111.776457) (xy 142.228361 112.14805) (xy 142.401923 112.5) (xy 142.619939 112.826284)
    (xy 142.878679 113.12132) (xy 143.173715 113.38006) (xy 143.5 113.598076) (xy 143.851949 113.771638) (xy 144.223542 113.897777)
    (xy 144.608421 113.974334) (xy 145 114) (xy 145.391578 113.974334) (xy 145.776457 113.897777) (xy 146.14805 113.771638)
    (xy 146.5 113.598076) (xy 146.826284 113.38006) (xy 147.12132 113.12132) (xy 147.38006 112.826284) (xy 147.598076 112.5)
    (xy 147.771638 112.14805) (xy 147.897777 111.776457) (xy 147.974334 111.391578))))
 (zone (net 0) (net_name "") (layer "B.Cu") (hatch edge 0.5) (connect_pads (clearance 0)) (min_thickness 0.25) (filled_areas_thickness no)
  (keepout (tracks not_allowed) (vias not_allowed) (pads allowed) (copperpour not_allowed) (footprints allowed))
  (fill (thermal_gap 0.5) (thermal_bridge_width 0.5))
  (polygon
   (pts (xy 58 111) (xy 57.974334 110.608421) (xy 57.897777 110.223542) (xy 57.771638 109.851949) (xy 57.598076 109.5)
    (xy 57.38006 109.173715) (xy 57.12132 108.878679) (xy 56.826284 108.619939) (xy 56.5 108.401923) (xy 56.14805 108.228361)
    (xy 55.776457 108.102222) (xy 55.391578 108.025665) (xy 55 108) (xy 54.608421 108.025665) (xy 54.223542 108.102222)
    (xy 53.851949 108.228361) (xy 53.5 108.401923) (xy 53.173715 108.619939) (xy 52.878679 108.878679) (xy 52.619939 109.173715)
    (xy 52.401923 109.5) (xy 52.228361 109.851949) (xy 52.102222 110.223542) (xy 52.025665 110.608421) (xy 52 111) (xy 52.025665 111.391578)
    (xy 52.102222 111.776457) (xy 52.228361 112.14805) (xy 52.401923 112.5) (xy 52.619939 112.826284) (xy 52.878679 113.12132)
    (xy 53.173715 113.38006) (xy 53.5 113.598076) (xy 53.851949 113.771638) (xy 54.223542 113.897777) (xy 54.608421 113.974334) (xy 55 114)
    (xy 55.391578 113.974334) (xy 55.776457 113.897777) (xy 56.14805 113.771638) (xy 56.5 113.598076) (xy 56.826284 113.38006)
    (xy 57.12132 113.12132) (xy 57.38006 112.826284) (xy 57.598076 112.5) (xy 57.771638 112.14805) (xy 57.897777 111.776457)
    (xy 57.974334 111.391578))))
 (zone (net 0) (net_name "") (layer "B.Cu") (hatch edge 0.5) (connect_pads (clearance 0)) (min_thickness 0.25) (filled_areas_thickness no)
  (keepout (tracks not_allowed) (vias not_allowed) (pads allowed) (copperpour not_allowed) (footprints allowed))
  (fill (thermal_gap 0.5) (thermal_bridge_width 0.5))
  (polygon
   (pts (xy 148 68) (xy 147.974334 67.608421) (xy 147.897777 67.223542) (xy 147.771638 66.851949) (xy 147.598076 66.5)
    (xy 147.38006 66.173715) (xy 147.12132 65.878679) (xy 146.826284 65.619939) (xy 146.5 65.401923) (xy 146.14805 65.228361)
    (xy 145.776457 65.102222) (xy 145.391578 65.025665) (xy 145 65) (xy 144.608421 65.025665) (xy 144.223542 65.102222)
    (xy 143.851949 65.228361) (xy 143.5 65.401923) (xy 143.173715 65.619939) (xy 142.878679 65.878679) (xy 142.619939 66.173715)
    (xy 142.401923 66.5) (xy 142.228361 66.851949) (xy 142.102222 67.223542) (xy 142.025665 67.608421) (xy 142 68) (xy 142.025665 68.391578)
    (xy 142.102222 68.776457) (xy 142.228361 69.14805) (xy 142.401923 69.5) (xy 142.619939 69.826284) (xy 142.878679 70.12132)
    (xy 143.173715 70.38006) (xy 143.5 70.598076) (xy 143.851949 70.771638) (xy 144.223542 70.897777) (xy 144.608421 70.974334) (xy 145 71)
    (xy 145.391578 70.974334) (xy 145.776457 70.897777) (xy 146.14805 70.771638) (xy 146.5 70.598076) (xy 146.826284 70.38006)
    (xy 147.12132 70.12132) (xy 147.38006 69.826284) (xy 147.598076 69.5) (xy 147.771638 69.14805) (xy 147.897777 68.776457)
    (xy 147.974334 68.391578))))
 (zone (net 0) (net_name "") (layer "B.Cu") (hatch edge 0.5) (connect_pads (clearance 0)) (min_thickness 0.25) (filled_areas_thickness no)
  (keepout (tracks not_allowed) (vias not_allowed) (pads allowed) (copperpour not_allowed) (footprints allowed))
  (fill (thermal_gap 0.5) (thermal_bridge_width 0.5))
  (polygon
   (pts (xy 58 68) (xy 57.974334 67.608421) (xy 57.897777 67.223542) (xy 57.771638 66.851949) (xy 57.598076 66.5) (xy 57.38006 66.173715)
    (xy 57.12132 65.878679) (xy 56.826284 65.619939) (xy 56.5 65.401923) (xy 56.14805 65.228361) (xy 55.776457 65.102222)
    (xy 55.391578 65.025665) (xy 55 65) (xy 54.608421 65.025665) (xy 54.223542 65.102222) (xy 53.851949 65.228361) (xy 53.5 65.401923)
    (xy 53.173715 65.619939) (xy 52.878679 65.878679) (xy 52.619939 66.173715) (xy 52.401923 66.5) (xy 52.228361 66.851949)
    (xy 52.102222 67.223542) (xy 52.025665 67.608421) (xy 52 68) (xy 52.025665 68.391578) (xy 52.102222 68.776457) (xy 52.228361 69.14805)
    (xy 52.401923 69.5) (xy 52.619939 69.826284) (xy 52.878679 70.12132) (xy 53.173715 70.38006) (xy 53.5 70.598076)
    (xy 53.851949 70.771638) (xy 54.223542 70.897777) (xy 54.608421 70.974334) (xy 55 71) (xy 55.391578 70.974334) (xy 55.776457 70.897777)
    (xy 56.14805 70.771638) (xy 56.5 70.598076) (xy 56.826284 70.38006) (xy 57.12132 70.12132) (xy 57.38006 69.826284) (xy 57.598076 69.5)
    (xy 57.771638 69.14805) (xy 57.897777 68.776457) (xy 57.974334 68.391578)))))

